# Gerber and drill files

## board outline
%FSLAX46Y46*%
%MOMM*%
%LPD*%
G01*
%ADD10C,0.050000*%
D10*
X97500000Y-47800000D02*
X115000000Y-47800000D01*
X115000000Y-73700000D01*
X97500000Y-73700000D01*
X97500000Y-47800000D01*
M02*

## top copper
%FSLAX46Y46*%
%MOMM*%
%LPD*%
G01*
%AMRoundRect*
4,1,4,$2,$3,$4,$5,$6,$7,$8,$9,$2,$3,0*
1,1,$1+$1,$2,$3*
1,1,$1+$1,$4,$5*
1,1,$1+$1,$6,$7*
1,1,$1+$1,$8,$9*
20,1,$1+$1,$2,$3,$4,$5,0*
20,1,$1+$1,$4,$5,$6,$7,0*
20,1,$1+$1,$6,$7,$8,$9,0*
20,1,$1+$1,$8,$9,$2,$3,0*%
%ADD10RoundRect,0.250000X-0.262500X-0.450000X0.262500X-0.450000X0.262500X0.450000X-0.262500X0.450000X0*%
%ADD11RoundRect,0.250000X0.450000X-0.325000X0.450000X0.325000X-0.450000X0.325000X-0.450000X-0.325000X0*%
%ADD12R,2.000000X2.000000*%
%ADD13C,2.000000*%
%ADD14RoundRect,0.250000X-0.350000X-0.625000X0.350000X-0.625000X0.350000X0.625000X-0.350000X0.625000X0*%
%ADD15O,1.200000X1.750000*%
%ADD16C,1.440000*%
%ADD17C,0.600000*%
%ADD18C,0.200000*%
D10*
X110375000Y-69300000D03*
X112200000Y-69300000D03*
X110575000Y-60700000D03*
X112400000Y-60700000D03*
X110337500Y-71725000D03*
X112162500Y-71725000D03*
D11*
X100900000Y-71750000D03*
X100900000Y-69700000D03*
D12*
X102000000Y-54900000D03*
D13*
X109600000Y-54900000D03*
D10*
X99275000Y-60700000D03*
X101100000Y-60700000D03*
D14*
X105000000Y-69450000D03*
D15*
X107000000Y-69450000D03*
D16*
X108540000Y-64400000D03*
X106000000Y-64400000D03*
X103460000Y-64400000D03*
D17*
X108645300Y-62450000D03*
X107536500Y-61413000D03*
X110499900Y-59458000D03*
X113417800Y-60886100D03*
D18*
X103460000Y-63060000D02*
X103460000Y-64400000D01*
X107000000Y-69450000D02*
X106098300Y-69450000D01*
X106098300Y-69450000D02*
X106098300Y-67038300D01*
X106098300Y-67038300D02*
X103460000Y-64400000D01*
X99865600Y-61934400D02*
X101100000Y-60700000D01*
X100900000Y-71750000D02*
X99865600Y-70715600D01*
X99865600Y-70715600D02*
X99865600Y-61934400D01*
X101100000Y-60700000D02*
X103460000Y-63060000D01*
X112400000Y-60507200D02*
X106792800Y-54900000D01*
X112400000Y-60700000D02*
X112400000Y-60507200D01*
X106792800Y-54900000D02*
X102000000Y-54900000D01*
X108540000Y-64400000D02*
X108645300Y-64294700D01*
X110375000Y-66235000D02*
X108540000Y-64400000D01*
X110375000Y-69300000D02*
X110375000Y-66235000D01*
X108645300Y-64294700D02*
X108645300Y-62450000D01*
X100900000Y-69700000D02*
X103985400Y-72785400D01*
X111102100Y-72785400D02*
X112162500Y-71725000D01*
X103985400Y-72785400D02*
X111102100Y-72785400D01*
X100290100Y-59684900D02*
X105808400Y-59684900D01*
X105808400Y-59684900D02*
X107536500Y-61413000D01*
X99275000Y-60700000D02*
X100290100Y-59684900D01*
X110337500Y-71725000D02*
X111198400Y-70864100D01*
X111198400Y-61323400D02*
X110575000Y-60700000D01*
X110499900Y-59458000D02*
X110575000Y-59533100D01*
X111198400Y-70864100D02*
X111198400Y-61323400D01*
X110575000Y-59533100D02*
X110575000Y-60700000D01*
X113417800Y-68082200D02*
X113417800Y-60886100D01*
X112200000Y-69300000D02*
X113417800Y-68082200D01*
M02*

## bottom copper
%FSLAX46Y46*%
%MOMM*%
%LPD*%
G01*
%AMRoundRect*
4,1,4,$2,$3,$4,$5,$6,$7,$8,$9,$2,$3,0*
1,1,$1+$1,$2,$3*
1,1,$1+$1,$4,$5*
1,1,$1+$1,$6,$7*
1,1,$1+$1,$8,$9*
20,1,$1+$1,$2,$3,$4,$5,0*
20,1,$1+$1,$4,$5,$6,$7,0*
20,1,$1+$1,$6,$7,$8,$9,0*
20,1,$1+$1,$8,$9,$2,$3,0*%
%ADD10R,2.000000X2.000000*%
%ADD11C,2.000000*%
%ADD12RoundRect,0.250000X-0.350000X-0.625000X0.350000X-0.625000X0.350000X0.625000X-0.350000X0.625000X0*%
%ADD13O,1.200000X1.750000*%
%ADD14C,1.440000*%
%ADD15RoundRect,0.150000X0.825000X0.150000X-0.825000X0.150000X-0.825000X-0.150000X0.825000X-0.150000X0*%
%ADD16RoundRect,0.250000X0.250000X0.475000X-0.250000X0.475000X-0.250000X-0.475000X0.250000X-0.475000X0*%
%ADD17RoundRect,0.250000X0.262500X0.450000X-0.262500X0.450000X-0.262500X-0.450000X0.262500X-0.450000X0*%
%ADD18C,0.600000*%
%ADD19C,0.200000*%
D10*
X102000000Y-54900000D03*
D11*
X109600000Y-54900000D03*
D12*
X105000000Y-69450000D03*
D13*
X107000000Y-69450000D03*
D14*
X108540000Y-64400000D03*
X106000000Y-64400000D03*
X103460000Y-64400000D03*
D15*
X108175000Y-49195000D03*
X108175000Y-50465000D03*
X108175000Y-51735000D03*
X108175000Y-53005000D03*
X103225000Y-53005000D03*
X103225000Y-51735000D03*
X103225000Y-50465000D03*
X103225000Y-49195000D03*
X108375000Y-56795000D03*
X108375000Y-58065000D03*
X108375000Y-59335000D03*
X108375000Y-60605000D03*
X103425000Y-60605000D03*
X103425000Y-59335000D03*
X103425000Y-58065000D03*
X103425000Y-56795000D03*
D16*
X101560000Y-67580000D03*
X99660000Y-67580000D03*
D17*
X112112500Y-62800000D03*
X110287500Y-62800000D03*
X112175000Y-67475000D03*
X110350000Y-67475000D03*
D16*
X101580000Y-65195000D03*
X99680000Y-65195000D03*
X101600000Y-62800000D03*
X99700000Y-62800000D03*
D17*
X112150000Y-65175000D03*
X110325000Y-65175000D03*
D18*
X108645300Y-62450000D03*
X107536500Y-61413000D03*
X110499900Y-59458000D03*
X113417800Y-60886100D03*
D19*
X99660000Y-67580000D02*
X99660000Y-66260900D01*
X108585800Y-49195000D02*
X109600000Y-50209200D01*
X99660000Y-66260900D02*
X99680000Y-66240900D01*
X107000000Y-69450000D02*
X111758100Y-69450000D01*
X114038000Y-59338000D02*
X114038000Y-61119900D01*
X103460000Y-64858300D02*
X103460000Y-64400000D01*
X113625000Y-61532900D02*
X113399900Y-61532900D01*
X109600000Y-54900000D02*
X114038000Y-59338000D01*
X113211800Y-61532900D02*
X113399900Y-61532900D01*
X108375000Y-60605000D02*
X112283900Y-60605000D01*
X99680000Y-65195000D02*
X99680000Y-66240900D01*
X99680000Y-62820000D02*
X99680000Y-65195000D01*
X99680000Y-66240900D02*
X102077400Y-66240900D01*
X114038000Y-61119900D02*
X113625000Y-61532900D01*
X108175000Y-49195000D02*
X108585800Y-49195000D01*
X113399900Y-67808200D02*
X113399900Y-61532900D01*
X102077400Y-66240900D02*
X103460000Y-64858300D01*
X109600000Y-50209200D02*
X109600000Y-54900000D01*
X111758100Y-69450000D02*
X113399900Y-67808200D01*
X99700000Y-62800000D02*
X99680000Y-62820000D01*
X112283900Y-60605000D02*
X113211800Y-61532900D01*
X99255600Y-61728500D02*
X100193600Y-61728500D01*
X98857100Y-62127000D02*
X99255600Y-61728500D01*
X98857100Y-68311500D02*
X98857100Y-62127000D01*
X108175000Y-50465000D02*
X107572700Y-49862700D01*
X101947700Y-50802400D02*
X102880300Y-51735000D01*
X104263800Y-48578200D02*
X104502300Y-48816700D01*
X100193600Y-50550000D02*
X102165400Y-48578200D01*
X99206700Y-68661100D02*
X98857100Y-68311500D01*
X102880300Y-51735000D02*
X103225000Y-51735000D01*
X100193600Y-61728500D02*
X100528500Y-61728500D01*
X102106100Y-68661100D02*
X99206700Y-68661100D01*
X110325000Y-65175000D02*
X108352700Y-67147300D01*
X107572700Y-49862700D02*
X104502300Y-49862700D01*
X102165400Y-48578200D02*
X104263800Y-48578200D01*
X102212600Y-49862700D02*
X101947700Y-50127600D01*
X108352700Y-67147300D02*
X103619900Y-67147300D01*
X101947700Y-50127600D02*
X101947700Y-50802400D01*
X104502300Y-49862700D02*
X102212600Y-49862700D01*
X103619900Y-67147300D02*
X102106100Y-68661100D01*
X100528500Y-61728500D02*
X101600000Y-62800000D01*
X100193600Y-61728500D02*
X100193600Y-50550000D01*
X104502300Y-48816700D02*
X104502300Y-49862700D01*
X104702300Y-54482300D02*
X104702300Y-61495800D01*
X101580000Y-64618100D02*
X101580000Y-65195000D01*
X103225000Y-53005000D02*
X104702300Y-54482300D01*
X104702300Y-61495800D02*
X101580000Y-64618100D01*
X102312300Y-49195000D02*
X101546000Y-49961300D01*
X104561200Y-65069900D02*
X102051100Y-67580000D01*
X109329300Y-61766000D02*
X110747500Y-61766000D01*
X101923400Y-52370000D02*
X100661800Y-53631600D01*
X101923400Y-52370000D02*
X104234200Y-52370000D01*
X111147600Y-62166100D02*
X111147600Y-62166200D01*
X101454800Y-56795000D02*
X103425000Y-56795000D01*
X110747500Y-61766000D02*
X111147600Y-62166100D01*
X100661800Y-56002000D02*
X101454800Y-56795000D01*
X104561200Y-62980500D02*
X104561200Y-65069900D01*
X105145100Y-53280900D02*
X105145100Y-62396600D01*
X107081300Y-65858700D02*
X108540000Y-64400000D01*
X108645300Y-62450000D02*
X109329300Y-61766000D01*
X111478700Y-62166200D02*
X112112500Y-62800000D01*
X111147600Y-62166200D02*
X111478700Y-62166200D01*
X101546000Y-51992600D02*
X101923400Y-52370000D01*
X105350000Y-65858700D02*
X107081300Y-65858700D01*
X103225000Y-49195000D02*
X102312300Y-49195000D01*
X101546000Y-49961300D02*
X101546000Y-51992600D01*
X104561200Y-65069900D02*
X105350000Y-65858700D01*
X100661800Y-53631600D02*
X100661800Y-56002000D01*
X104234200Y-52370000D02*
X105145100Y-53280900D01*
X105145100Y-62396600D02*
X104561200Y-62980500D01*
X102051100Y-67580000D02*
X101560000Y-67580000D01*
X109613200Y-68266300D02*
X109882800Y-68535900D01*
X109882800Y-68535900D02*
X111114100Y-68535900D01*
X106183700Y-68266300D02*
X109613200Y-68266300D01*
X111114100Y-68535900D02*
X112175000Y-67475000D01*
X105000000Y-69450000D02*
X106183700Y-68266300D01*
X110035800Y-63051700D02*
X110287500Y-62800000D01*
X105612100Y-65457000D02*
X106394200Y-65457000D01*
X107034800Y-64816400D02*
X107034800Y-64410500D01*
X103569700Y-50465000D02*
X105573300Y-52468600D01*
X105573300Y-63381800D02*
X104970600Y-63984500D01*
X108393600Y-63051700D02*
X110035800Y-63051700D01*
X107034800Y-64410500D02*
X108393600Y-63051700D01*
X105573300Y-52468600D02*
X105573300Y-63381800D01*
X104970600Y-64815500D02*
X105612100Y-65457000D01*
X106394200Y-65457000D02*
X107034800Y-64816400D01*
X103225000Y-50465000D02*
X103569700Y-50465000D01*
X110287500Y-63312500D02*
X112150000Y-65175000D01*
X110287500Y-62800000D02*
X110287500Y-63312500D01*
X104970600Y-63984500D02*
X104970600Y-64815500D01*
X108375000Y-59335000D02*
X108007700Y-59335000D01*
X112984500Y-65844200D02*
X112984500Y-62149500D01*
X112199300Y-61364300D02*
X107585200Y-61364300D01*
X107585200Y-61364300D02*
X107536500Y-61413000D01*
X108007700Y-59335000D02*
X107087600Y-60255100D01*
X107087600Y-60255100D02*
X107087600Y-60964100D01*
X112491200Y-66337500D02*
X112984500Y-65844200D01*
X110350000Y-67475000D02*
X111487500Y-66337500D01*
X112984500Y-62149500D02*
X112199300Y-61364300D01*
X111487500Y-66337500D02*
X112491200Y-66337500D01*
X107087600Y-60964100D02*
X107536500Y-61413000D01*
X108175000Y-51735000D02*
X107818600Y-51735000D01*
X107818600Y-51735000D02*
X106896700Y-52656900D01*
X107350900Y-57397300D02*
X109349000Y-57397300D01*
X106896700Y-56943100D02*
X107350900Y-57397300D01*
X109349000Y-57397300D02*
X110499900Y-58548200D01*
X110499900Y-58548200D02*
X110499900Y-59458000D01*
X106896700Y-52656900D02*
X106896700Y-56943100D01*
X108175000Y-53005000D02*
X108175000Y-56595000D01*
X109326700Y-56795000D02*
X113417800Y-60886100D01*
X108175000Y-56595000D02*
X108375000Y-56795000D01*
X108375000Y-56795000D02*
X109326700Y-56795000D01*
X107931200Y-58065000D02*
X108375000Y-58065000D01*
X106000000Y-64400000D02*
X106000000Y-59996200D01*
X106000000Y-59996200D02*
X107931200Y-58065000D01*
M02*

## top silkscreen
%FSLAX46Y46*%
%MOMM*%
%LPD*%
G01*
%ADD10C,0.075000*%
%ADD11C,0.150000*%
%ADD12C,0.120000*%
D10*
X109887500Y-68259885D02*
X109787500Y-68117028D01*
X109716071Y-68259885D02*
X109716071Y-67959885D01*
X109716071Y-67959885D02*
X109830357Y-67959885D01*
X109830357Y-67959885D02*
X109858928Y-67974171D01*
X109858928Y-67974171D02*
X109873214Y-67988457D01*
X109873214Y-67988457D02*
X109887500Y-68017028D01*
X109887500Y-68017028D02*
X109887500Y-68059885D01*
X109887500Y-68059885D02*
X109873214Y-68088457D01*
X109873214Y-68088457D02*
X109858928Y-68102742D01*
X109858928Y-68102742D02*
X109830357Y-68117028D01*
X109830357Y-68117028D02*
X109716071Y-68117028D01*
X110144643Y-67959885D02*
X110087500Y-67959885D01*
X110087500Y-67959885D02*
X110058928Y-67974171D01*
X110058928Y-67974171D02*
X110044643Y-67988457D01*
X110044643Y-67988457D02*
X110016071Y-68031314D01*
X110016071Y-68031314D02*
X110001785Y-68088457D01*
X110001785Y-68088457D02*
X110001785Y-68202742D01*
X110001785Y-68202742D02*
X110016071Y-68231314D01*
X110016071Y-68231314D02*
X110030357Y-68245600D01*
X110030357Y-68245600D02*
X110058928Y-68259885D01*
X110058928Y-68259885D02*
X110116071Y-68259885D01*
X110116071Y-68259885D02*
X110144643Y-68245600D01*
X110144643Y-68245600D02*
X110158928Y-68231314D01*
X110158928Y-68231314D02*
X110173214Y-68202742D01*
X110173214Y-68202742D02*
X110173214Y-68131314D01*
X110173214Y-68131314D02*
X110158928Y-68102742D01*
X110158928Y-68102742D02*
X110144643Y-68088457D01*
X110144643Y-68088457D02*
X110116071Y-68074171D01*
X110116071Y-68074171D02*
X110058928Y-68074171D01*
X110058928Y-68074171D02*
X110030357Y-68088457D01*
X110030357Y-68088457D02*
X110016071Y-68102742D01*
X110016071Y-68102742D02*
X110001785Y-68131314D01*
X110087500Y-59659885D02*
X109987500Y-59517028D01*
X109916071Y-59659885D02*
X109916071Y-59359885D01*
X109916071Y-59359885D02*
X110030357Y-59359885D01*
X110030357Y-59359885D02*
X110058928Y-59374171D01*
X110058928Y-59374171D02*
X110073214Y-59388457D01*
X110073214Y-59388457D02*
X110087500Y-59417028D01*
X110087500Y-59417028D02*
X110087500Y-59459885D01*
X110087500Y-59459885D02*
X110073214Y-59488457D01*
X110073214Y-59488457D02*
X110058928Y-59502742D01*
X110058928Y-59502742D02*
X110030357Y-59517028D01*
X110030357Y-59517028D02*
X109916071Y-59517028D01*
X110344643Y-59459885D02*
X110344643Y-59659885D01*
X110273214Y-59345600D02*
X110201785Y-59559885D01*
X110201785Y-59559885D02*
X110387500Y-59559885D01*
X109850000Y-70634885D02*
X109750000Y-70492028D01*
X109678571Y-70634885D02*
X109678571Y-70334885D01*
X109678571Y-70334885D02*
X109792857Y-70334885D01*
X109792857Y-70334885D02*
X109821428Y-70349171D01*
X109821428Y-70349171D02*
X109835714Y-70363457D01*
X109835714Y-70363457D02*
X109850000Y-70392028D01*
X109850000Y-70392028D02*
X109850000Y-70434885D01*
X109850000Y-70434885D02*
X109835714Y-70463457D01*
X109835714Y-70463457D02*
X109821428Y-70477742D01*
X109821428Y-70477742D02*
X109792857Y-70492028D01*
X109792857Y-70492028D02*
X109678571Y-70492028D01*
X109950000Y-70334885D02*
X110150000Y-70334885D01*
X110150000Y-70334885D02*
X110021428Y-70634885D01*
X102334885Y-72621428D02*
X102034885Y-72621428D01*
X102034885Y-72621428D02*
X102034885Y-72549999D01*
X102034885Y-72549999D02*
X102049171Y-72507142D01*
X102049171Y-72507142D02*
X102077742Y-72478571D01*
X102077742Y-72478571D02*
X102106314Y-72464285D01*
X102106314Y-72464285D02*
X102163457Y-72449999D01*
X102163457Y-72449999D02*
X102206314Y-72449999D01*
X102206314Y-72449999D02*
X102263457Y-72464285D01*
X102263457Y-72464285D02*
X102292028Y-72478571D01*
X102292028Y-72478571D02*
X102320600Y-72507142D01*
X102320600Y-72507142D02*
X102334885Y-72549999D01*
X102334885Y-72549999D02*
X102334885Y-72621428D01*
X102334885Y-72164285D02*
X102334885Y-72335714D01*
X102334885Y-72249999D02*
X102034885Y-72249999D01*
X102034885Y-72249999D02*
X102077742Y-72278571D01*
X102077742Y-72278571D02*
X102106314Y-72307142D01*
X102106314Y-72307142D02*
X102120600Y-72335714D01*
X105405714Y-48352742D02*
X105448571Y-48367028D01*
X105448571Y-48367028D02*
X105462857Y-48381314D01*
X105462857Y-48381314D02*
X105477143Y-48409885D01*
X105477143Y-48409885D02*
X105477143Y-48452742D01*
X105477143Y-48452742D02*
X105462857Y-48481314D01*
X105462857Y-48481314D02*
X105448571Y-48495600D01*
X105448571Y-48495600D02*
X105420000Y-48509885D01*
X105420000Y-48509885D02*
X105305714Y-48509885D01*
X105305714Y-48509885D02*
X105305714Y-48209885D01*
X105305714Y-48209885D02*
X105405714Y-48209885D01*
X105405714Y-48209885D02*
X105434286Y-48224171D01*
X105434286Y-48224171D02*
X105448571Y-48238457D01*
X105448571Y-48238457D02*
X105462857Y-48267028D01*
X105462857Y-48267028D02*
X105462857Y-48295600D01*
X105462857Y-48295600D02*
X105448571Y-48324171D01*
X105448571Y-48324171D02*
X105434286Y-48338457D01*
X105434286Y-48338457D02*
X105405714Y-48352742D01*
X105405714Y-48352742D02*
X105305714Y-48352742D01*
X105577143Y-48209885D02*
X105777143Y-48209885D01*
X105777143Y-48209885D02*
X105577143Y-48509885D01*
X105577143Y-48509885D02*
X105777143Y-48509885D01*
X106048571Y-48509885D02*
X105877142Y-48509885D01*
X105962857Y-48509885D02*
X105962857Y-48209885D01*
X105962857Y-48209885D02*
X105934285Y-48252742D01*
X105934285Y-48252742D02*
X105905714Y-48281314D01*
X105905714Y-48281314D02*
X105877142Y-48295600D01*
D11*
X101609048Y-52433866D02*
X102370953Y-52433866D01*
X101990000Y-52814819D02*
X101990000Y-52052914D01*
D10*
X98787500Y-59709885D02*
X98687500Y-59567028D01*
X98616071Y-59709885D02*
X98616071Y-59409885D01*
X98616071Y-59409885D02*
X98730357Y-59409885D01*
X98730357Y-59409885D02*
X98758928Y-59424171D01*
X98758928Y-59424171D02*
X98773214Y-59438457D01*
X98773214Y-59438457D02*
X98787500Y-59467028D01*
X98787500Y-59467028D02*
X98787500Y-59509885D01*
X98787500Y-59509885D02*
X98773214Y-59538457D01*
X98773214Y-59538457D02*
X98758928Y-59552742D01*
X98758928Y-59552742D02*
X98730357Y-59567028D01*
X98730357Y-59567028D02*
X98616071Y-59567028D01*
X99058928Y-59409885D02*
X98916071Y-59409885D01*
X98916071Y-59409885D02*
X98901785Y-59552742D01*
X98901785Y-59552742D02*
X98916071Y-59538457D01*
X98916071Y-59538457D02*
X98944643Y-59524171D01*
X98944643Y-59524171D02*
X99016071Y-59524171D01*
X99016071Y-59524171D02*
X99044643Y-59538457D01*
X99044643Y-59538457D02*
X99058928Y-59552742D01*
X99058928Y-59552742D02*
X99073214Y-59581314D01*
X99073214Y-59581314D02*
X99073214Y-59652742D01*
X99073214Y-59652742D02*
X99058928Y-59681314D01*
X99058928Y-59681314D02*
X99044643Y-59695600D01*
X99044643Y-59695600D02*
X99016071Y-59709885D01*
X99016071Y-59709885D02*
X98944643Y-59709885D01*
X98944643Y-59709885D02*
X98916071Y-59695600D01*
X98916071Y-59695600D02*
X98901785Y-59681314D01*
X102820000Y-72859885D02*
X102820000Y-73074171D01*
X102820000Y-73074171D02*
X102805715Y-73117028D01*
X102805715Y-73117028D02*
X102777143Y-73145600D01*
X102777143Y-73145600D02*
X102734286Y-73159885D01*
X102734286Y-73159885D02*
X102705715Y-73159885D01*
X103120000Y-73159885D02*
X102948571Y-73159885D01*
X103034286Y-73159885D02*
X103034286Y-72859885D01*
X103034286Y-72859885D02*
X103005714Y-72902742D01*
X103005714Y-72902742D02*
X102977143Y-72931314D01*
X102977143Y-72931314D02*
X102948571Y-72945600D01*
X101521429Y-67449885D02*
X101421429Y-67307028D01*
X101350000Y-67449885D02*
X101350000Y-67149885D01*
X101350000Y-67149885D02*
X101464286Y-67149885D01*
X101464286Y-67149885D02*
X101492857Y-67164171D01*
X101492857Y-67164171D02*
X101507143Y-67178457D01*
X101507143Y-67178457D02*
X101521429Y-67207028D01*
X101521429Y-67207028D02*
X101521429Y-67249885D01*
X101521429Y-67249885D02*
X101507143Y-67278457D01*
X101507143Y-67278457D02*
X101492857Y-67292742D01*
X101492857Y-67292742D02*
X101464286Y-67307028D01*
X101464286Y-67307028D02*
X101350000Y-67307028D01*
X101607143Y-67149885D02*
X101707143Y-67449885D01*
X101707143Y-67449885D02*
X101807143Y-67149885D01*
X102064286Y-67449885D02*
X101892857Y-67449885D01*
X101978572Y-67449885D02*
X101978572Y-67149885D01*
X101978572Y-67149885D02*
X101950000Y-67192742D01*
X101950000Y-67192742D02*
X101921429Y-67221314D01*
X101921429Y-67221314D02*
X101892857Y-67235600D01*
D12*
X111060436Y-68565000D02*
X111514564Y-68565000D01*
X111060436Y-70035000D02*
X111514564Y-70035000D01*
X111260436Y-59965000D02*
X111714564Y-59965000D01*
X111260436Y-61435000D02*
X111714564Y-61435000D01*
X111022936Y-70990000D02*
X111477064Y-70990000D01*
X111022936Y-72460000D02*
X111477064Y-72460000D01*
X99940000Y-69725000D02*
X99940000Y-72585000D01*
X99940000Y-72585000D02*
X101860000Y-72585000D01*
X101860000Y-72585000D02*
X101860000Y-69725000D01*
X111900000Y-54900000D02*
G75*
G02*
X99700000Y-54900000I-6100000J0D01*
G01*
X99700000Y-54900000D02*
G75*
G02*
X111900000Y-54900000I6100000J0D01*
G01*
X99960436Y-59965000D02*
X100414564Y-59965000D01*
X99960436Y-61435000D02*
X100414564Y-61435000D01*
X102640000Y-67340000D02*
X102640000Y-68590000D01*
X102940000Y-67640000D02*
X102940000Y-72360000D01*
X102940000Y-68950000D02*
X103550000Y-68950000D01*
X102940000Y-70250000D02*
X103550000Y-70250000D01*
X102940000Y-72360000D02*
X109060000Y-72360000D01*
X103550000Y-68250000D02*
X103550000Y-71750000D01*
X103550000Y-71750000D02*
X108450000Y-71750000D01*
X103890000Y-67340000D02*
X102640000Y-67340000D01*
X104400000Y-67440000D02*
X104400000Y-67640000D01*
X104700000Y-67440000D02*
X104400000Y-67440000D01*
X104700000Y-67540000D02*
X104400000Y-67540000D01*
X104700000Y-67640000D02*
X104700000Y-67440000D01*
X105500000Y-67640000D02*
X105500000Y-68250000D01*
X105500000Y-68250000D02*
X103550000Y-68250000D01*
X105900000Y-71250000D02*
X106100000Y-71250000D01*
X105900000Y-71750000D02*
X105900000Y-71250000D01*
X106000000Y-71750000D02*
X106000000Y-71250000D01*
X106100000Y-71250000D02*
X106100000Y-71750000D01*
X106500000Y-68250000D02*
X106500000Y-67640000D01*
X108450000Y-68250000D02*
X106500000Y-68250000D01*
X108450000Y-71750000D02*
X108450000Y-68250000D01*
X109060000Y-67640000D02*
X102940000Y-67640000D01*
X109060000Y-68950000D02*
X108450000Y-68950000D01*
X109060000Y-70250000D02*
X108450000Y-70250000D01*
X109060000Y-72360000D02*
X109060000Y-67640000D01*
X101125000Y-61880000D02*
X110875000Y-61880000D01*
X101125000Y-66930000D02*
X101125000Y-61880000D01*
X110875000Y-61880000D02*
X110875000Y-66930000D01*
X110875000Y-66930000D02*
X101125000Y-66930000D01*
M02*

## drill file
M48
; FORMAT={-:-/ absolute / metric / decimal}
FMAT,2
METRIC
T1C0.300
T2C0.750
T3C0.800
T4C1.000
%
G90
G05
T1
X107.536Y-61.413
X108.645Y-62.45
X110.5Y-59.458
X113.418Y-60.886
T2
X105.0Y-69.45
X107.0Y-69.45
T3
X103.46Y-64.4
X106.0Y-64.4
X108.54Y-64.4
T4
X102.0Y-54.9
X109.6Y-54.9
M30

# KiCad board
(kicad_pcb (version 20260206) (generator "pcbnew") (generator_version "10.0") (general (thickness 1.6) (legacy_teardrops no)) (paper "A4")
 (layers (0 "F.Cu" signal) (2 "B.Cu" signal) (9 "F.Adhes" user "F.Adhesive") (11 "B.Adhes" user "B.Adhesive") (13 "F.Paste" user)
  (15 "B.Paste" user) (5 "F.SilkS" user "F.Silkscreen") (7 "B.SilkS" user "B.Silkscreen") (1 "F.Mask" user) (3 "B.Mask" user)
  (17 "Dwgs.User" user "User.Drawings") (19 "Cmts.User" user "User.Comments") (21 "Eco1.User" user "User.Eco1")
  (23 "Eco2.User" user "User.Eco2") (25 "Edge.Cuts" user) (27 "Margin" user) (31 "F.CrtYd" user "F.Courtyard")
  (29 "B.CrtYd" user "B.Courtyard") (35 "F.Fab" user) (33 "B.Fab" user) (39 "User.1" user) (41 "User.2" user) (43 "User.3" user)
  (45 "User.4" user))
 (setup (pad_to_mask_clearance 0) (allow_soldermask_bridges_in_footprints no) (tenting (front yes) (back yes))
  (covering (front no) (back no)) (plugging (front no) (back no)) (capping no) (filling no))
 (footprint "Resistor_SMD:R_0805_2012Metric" (layer "F.Cu") (at 111.2875 69.3)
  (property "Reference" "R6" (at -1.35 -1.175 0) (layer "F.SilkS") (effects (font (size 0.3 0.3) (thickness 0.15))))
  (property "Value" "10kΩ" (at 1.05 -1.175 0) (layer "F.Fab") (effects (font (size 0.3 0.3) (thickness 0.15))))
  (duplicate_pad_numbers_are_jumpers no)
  (fp_line (start -0.227064 -0.735) (end 0.227064 -0.735) (stroke (width 0.12) (type solid)) (layer "F.SilkS"))
  (fp_line (start -0.227064 0.735) (end 0.227064 0.735) (stroke (width 0.12) (type solid)) (layer "F.SilkS"))
  (pad "1" smd roundrect (at -0.9125 0) (size 1.025 1.4) (layers "F.Cu" "F.Mask" "F.Paste") (roundrect_rratio 0.243902) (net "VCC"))
  (pad "2" smd roundrect (at 0.9125 0) (size 1.025 1.4) (layers "F.Cu" "F.Mask" "F.Paste") (roundrect_rratio 0.243902) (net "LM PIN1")))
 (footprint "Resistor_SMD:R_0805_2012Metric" (layer "F.Cu") (at 111.4875 60.7)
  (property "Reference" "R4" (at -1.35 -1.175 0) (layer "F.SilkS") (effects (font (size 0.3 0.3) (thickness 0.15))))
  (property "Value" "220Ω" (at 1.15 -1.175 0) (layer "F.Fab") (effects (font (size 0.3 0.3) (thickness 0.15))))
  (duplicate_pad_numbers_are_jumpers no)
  (fp_line (start -0.227064 -0.735) (end 0.227064 -0.735) (stroke (width 0.12) (type solid)) (layer "F.SilkS"))
  (fp_line (start -0.227064 0.735) (end 0.227064 0.735) (stroke (width 0.12) (type solid)) (layer "F.SilkS"))
  (pad "1" smd roundrect (at -0.9125 0) (size 1.025 1.4) (layers "F.Cu" "F.Mask" "F.Paste") (roundrect_rratio 0.243902) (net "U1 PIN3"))
  (pad "2" smd roundrect (at 0.9125 0) (size 1.025 1.4) (layers "F.Cu" "F.Mask" "F.Paste") (roundrect_rratio 0.243902) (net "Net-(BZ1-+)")))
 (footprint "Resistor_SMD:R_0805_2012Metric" (layer "F.Cu") (at 111.25 71.725)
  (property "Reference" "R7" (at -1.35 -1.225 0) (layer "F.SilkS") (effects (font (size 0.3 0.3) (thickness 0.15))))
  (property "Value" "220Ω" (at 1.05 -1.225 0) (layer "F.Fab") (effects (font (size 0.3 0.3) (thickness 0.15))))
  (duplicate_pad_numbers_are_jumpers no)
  (fp_line (start -0.227064 -0.735) (end 0.227064 -0.735) (stroke (width 0.12) (type solid)) (layer "F.SilkS"))
  (fp_line (start -0.227064 0.735) (end 0.227064 0.735) (stroke (width 0.12) (type solid)) (layer "F.SilkS"))
  (pad "1" smd roundrect (at -0.9125 0) (size 1.025 1.4) (layers "F.Cu" "F.Mask" "F.Paste") (roundrect_rratio 0.243902) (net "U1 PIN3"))
  (pad "2" smd roundrect (at 0.9125 0) (size 1.025 1.4) (layers "F.Cu" "F.Mask" "F.Paste") (roundrect_rratio 0.243902) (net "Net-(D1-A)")))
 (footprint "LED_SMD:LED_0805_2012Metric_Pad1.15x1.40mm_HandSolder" (layer "F.Cu") (at 100.9 70.725 90)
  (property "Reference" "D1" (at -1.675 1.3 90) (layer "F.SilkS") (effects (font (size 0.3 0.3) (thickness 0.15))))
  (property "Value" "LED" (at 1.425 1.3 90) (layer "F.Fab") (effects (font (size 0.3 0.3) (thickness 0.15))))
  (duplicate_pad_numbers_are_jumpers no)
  (fp_line (start 1 -0.96) (end -1.86 -0.96) (stroke (width 0.12) (type solid)) (layer "F.SilkS"))
  (fp_line (start -1.86 -0.96) (end -1.86 0.96) (stroke (width 0.12) (type solid)) (layer "F.SilkS"))
  (fp_line (start -1.86 0.96) (end 1 0.96) (stroke (width 0.12) (type solid)) (layer "F.SilkS"))
  (pad "1" smd roundrect (at -1.025 0 90) (size 1.15 1.4) (layers "F.Cu" "F.Mask" "F.Paste") (roundrect_rratio 0.217391) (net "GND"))
  (pad "2" smd roundrect (at 1.025 0 90) (size 1.15 1.4) (layers "F.Cu" "F.Mask" "F.Paste") (roundrect_rratio 0.217391) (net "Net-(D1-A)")))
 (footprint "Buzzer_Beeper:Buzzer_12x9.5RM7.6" (layer "F.Cu") (at 102 54.9)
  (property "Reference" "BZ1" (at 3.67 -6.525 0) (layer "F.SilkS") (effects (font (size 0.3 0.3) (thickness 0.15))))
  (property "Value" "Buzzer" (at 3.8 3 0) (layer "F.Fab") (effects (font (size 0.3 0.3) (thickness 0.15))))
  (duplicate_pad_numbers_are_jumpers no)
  (fp_circle (center 3.8 0) (end 9.9 0) (stroke (width 0.12) (type solid)) (fill no) (layer "F.SilkS"))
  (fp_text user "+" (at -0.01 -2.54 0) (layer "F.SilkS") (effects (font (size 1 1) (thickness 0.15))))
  (pad "1" thru_hole rect (at 0 0) (size 2 2) (drill 1) (layers "*.Cu" "*.Mask") (remove_unused_layers no) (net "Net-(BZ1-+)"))
  (pad "2" thru_hole circle (at 7.6 0) (size 2 2) (drill 1) (layers "*.Cu" "*.Mask") (remove_unused_layers no) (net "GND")))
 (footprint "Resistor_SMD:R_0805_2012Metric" (layer "F.Cu") (at 100.1875 60.7)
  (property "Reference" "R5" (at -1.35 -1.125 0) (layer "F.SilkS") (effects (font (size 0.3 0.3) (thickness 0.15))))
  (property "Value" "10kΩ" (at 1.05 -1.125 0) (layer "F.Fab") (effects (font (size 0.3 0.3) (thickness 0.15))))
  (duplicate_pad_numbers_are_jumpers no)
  (fp_line (start -0.227064 -0.735) (end 0.227064 -0.735) (stroke (width 0.12) (type solid)) (layer "F.SilkS"))
  (fp_line (start -0.227064 0.735) (end 0.227064 0.735) (stroke (width 0.12) (type solid)) (layer "F.SilkS"))
  (pad "1" smd roundrect (at -0.9125 0) (size 1.025 1.4) (layers "F.Cu" "F.Mask" "F.Paste") (roundrect_rratio 0.243902)
   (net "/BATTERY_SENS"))
  (pad "2" smd roundrect (at 0.9125 0) (size 1.025 1.4) (layers "F.Cu" "F.Mask" "F.Paste") (roundrect_rratio 0.243902) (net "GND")))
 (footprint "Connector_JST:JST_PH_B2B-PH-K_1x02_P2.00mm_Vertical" (layer "F.Cu") (at 105 69.45)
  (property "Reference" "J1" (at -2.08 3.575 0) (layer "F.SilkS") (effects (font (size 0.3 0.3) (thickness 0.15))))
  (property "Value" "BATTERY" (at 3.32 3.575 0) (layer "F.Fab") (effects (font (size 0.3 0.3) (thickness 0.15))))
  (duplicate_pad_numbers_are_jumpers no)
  (fp_line (start -2.36 -2.11) (end -2.36 -0.86) (stroke (width 0.12) (type solid)) (layer "F.SilkS"))
  (fp_line (start -2.06 -1.81) (end -2.06 2.91) (stroke (width 0.12) (type solid)) (layer "F.SilkS"))
  (fp_line (start -2.06 -0.5) (end -1.45 -0.5) (stroke (width 0.12) (type solid)) (layer "F.SilkS"))
  (fp_line (start -2.06 0.8) (end -1.45 0.8) (stroke (width 0.12) (type solid)) (layer "F.SilkS"))
  (fp_line (start -2.06 2.91) (end 4.06 2.91) (stroke (width 0.12) (type solid)) (layer "F.SilkS"))
  (fp_line (start -1.45 -1.2) (end -1.45 2.3) (stroke (width 0.12) (type solid)) (layer "F.SilkS"))
  (fp_line (start -1.45 2.3) (end 3.45 2.3) (stroke (width 0.12) (type solid)) (layer "F.SilkS"))
  (fp_line (start -1.11 -2.11) (end -2.36 -2.11) (stroke (width 0.12) (type solid)) (layer "F.SilkS"))
  (fp_line (start -0.6 -2.01) (end -0.6 -1.81) (stroke (width 0.12) (type solid)) (layer "F.SilkS"))
  (fp_line (start -0.3 -2.01) (end -0.6 -2.01) (stroke (width 0.12) (type solid)) (layer "F.SilkS"))
  (fp_line (start -0.3 -1.91) (end -0.6 -1.91) (stroke (width 0.12) (type solid)) (layer "F.SilkS"))
  (fp_line (start -0.3 -1.81) (end -0.3 -2.01) (stroke (width 0.12) (type solid)) (layer "F.SilkS"))
  (fp_line (start 0.5 -1.81) (end 0.5 -1.2) (stroke (width 0.12) (type solid)) (layer "F.SilkS"))
  (fp_line (start 0.5 -1.2) (end -1.45 -1.2) (stroke (width 0.12) (type solid)) (layer "F.SilkS"))
  (fp_line (start 0.9 1.8) (end 1.1 1.8) (stroke (width 0.12) (type solid)) (layer "F.SilkS"))
  (fp_line (start 0.9 2.3) (end 0.9 1.8) (stroke (width 0.12) (type solid)) (layer "F.SilkS"))
  (fp_line (start 1 2.3) (end 1 1.8) (stroke (width 0.12) (type solid)) (layer "F.SilkS"))
  (fp_line (start 1.1 1.8) (end 1.1 2.3) (stroke (width 0.12) (type solid)) (layer "F.SilkS"))
  (fp_line (start 1.5 -1.2) (end 1.5 -1.81) (stroke (width 0.12) (type solid)) (layer "F.SilkS"))
  (fp_line (start 3.45 -1.2) (end 1.5 -1.2) (stroke (width 0.12) (type solid)) (layer "F.SilkS"))
  (fp_line (start 3.45 2.3) (end 3.45 -1.2) (stroke (width 0.12) (type solid)) (layer "F.SilkS"))
  (fp_line (start 4.06 -1.81) (end -2.06 -1.81) (stroke (width 0.12) (type solid)) (layer "F.SilkS"))
  (fp_line (start 4.06 -0.5) (end 3.45 -0.5) (stroke (width 0.12) (type solid)) (layer "F.SilkS"))
  (fp_line (start 4.06 0.8) (end 3.45 0.8) (stroke (width 0.12) (type solid)) (layer "F.SilkS"))
  (fp_line (start 4.06 2.91) (end 4.06 -1.81) (stroke (width 0.12) (type solid)) (layer "F.SilkS"))
  (pad "1" thru_hole roundrect (at 0 0) (size 1.2 1.75) (drill 0.75) (layers "*.Cu" "*.Mask") (remove_unused_layers no)
   (roundrect_rratio 0.208333) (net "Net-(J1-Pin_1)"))
  (pad "2" thru_hole oval (at 2 0) (size 1.2 1.75) (drill 0.75) (layers "*.Cu" "*.Mask") (remove_unused_layers no) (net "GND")))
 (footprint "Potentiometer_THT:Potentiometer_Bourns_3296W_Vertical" (layer "F.Cu") (at 108.54 64.4)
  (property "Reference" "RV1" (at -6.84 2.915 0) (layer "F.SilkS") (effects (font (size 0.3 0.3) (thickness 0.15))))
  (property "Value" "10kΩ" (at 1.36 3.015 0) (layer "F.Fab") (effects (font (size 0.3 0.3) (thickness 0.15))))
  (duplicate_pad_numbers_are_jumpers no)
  (fp_line (start -7.415 -2.52) (end 2.335 -2.52) (stroke (width 0.12) (type solid)) (layer "F.SilkS"))
  (fp_line (start -7.415 2.53) (end -7.415 -2.52) (stroke (width 0.12) (type solid)) (layer "F.SilkS"))
  (fp_line (start 2.335 -2.52) (end 2.335 2.53) (stroke (width 0.12) (type solid)) (layer "F.SilkS"))
  (fp_line (start 2.335 2.53) (end -7.415 2.53) (stroke (width 0.12) (type solid)) (layer "F.SilkS"))
  (pad "1" thru_hole circle (at 0 0) (size 1.44 1.44) (drill 0.8) (layers "*.Cu" "*.Mask") (remove_unused_layers no) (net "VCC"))
  (pad "2" thru_hole circle (at -2.54 0) (size 1.44 1.44) (drill 0.8) (layers "*.Cu" "*.Mask") (remove_unused_layers no) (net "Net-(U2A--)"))
  (pad "3" thru_hole circle (at -5.08 0) (size 1.44 1.44) (drill 0.8) (layers "*.Cu" "*.Mask") (remove_unused_layers no) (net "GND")))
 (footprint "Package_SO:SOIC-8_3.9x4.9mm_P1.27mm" (layer "B.Cu") (at 105.7 51.1 180)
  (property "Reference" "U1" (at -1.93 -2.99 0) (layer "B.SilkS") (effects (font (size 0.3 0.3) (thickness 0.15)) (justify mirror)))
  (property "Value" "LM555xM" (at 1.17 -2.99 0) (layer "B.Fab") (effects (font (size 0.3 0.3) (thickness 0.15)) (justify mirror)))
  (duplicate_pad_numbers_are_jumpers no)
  (pad "1" smd roundrect (at -2.475 1.905 180) (size 1.95 0.6) (layers "B.Cu" "B.Mask" "B.Paste") (roundrect_rratio 0.25) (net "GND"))
  (pad "2" smd roundrect (at -2.475 0.635 180) (size 1.95 0.6) (layers "B.Cu" "B.Mask" "B.Paste") (roundrect_rratio 0.25) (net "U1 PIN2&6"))
  (pad "3" smd roundrect (at -2.475 -0.635 180) (size 1.95 0.6) (layers "B.Cu" "B.Mask" "B.Paste") (roundrect_rratio 0.25) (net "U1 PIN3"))
  (pad "4" smd roundrect (at -2.475 -1.905 180) (size 1.95 0.6) (layers "B.Cu" "B.Mask" "B.Paste") (roundrect_rratio 0.25) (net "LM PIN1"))
  (pad "5" smd roundrect (at 2.475 -1.905 180) (size 1.95 0.6) (layers "B.Cu" "B.Mask" "B.Paste") (roundrect_rratio 0.25) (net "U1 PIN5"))
  (pad "6" smd roundrect (at 2.475 -0.635 180) (size 1.95 0.6) (layers "B.Cu" "B.Mask" "B.Paste") (roundrect_rratio 0.25) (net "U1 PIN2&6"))
  (pad "7" smd roundrect (at 2.475 0.635 180) (size 1.95 0.6) (layers "B.Cu" "B.Mask" "B.Paste") (roundrect_rratio 0.25) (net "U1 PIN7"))
  (pad "8" smd roundrect (at 2.475 1.905 180) (size 1.95 0.6) (layers "B.Cu" "B.Mask" "B.Paste") (roundrect_rratio 0.25) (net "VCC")))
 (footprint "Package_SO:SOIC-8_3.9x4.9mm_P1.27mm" (layer "B.Cu") (at 105.9 58.7 180)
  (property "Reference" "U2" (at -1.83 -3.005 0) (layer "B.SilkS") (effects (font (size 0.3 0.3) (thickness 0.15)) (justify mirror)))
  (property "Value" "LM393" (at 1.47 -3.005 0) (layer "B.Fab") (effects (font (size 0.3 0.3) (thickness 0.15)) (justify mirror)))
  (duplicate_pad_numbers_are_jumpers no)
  (pad "1" smd roundrect (at -2.475 1.905 180) (size 1.95 0.6) (layers "B.Cu" "B.Mask" "B.Paste") (roundrect_rratio 0.25) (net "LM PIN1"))
  (pad "2" smd roundrect (at -2.475 0.635 180) (size 1.95 0.6) (layers "B.Cu" "B.Mask" "B.Paste") (roundrect_rratio 0.25)
   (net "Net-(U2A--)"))
  (pad "3" smd roundrect (at -2.475 -0.635 180) (size 1.95 0.6) (layers "B.Cu" "B.Mask" "B.Paste") (roundrect_rratio 0.25)
   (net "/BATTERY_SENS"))
  (pad "4" smd roundrect (at -2.475 -1.905 180) (size 1.95 0.6) (layers "B.Cu" "B.Mask" "B.Paste") (roundrect_rratio 0.25) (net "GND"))
  (pad "5" smd roundrect (at 2.475 -1.905 180) (size 1.95 0.6) (layers "B.Cu" "B.Mask" "B.Paste") (roundrect_rratio 0.25)
   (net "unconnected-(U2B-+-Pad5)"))
  (pad "6" smd roundrect (at 2.475 -0.635 180) (size 1.95 0.6) (layers "B.Cu" "B.Mask" "B.Paste") (roundrect_rratio 0.25)
   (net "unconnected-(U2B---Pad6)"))
  (pad "7" smd roundrect (at 2.475 0.635 180) (size 1.95 0.6) (layers "B.Cu" "B.Mask" "B.Paste") (roundrect_rratio 0.25)
   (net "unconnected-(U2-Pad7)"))
  (pad "8" smd roundrect (at 2.475 1.905 180) (size 1.95 0.6) (layers "B.Cu" "B.Mask" "B.Paste") (roundrect_rratio 0.25) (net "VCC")))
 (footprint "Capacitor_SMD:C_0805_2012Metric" (layer "B.Cu") (at 100.61 67.58 180)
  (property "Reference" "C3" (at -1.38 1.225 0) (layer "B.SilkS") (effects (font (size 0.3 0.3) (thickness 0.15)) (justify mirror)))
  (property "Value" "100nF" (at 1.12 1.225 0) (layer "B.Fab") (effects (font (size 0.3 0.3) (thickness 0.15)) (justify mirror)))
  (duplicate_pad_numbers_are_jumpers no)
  (pad "1" smd roundrect (at -0.95 0 180) (size 1 1.45) (layers "B.Cu" "B.Mask" "B.Paste") (roundrect_rratio 0.25) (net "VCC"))
  (pad "2" smd roundrect (at 0.95 0 180) (size 1 1.45) (layers "B.Cu" "B.Mask" "B.Paste") (roundrect_rratio 0.25) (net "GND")))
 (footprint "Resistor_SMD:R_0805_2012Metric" (layer "B.Cu") (at 111.2 62.8 180)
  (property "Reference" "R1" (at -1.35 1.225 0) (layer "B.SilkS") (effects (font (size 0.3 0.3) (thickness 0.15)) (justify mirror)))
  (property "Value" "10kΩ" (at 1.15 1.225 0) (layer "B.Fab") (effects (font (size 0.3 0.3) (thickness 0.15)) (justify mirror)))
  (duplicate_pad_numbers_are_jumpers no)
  (pad "1" smd roundrect (at -0.9125 0 180) (size 1.025 1.4) (layers "B.Cu" "B.Mask" "B.Paste") (roundrect_rratio 0.243902) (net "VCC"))
  (pad "2" smd roundrect (at 0.9125 0 180) (size 1.025 1.4) (layers "B.Cu" "B.Mask" "B.Paste") (roundrect_rratio 0.243902) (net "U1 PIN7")))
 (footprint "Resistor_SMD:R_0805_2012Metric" (layer "B.Cu") (at 111.2625 67.475 180)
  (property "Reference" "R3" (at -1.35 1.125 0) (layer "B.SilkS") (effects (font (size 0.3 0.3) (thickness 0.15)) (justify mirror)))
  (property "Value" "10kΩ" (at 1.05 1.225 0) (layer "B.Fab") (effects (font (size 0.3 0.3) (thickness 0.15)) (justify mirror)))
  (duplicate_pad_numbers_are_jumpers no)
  (pad "1" smd roundrect (at -0.9125 0 180) (size 1.025 1.4) (layers "B.Cu" "B.Mask" "B.Paste") (roundrect_rratio 0.243902)
   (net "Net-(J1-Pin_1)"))
  (pad "2" smd roundrect (at 0.9125 0 180) (size 1.025 1.4) (layers "B.Cu" "B.Mask" "B.Paste") (roundrect_rratio 0.243902)
   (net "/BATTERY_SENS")))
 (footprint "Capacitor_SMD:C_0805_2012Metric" (layer "B.Cu") (at 100.63 65.195 180)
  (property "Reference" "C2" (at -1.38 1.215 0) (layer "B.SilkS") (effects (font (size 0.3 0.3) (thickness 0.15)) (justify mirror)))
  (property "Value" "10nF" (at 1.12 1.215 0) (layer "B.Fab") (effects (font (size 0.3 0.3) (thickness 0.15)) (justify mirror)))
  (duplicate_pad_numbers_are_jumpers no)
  (pad "1" smd roundrect (at -0.95 0 180) (size 1 1.45) (layers "B.Cu" "B.Mask" "B.Paste") (roundrect_rratio 0.25) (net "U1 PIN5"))
  (pad "2" smd roundrect (at 0.95 0 180) (size 1 1.45) (layers "B.Cu" "B.Mask" "B.Paste") (roundrect_rratio 0.25) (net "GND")))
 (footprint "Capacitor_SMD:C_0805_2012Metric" (layer "B.Cu") (at 100.65 62.8 180)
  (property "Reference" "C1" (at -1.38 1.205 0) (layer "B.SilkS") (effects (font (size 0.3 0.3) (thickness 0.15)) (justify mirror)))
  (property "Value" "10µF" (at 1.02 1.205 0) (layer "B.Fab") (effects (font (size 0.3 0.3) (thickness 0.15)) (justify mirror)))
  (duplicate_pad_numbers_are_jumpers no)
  (pad "1" smd roundrect (at -0.95 0 180) (size 1 1.45) (layers "B.Cu" "B.Mask" "B.Paste") (roundrect_rratio 0.25) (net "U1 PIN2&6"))
  (pad "2" smd roundrect (at 0.95 0 180) (size 1 1.45) (layers "B.Cu" "B.Mask" "B.Paste") (roundrect_rratio 0.25) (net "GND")))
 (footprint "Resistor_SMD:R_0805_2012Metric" (layer "B.Cu") (at 111.2375 65.175 180)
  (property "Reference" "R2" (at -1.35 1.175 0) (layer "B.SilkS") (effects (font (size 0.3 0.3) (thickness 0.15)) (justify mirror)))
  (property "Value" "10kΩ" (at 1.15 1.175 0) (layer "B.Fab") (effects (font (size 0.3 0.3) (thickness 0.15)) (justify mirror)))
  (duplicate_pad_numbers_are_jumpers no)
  (pad "1" smd roundrect (at -0.9125 0 180) (size 1.025 1.4) (layers "B.Cu" "B.Mask" "B.Paste") (roundrect_rratio 0.243902) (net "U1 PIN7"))
  (pad "2" smd roundrect (at 0.9125 0 180) (size 1.025 1.4) (layers "B.Cu" "B.Mask" "B.Paste") (roundrect_rratio 0.243902) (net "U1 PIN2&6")))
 (gr_rect (start 97.5 47.8) (end 115 73.7) (stroke (width 0.05) (type default)) (fill no) (layer "Edge.Cuts"))
 (segment (start 103.46 63.06) (end 103.46 64.4) (width 0.2) (layer "F.Cu") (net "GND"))
 (segment (start 107 69.45) (end 106.0983 69.45) (width 0.2) (layer "F.Cu") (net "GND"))
 (segment (start 106.0983 69.45) (end 106.0983 67.0383) (width 0.2) (layer "F.Cu") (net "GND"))
 (segment (start 106.0983 67.0383) (end 103.46 64.4) (width 0.2) (layer "F.Cu") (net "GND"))
 (segment (start 99.8656 61.9344) (end 101.1 60.7) (width 0.2) (layer "F.Cu") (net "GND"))
 (segment (start 100.9 71.75) (end 99.8656 70.7156) (width 0.2) (layer "F.Cu") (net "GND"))
 (segment (start 99.8656 70.7156) (end 99.8656 61.9344) (width 0.2) (layer "F.Cu") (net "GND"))
 (segment (start 101.1 60.7) (end 103.46 63.06) (width 0.2) (layer "F.Cu") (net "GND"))
 (segment (start 99.66 67.58) (end 99.66 66.2609) (width 0.2) (layer "B.Cu") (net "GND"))
 (segment (start 108.5858 49.195) (end 109.6 50.2092) (width 0.2) (layer "B.Cu") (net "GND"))
 (segment (start 99.66 66.2609) (end 99.68 66.2409) (width 0.2) (layer "B.Cu") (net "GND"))
 (segment (start 107 69.45) (end 111.7581 69.45) (width 0.2) (layer "B.Cu") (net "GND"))
 (segment (start 114.038 59.338) (end 114.038 61.1199) (width 0.2) (layer "B.Cu") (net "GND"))
 (segment (start 103.46 64.8583) (end 103.46 64.4) (width 0.2) (layer "B.Cu") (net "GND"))
 (segment (start 113.625 61.5329) (end 113.3999 61.5329) (width 0.2) (layer "B.Cu") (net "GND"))
 (segment (start 109.6 54.9) (end 114.038 59.338) (width 0.2) (layer "B.Cu") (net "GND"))
 (segment (start 113.2118 61.5329) (end 113.3999 61.5329) (width 0.2) (layer "B.Cu") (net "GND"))
 (segment (start 108.375 60.605) (end 112.2839 60.605) (width 0.2) (layer "B.Cu") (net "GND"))
 (segment (start 99.68 65.195) (end 99.68 66.2409) (width 0.2) (layer "B.Cu") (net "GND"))
 (segment (start 99.68 62.82) (end 99.68 65.195) (width 0.2) (layer "B.Cu") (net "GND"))
 (segment (start 99.68 66.2409) (end 102.0774 66.2409) (width 0.2) (layer "B.Cu") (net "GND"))
 (segment (start 114.038 61.1199) (end 113.625 61.5329) (width 0.2) (layer "B.Cu") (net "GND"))
 (segment (start 108.175 49.195) (end 108.5858 49.195) (width 0.2) (layer "B.Cu") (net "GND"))
 (segment (start 113.3999 67.8082) (end 113.3999 61.5329) (width 0.2) (layer "B.Cu") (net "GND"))
 (segment (start 102.0774 66.2409) (end 103.46 64.8583) (width 0.2) (layer "B.Cu") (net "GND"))
 (segment (start 109.6 50.2092) (end 109.6 54.9) (width 0.2) (layer "B.Cu") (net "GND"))
 (segment (start 111.7581 69.45) (end 113.3999 67.8082) (width 0.2) (layer "B.Cu") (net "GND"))
 (segment (start 99.7 62.8) (end 99.68 62.82) (width 0.2) (layer "B.Cu") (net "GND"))
 (segment (start 112.2839 60.605) (end 113.2118 61.5329) (width 0.2) (layer "B.Cu") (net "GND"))
 (segment (start 112.4 60.5072) (end 106.7928 54.9) (width 0.2) (layer "F.Cu") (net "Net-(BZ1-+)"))
 (segment (start 112.4 60.7) (end 112.4 60.5072) (width 0.2) (layer "F.Cu") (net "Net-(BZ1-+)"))
 (segment (start 106.7928 54.9) (end 102 54.9) (width 0.2) (layer "F.Cu") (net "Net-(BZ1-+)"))
 (segment (start 99.2556 61.7285) (end 100.1936 61.7285) (width 0.2) (layer "B.Cu") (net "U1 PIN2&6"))
 (segment (start 98.8571 62.127) (end 99.2556 61.7285) (width 0.2) (layer "B.Cu") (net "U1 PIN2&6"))
 (segment (start 98.8571 68.3115) (end 98.8571 62.127) (width 0.2) (layer "B.Cu") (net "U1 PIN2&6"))
 (segment (start 108.175 50.465) (end 107.5727 49.8627) (width 0.2) (layer "B.Cu") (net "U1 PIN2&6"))
 (segment (start 101.9477 50.8024) (end 102.8803 51.735) (width 0.2) (layer "B.Cu") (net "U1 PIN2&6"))
 (segment (start 104.2638 48.5782) (end 104.5023 48.8167) (width 0.2) (layer "B.Cu") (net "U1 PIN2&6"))
 (segment (start 100.1936 50.55) (end 102.1654 48.5782) (width 0.2) (layer "B.Cu") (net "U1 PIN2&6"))
 (segment (start 99.2067 68.6611) (end 98.8571 68.3115) (width 0.2) (layer "B.Cu") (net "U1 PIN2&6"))
 (segment (start 102.8803 51.735) (end 103.225 51.735) (width 0.2) (layer "B.Cu") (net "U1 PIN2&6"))
 (segment (start 100.1936 61.7285) (end 100.5285 61.7285) (width 0.2) (layer "B.Cu") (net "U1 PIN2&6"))
 (segment (start 102.1061 68.6611) (end 99.2067 68.6611) (width 0.2) (layer "B.Cu") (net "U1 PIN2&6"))
 (segment (start 110.325 65.175) (end 108.3527 67.1473) (width 0.2) (layer "B.Cu") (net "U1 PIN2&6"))
 (segment (start 107.5727 49.8627) (end 104.5023 49.8627) (width 0.2) (layer "B.Cu") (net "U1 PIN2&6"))
 (segment (start 102.1654 48.5782) (end 104.2638 48.5782) (width 0.2) (layer "B.Cu") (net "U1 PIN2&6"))
 (segment (start 102.2126 49.8627) (end 101.9477 50.1276) (width 0.2) (layer "B.Cu") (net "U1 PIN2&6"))
 (segment (start 108.3527 67.1473) (end 103.6199 67.1473) (width 0.2) (layer "B.Cu") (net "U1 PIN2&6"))
 (segment (start 101.9477 50.1276) (end 101.9477 50.8024) (width 0.2) (layer "B.Cu") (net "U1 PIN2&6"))
 (segment (start 104.5023 49.8627) (end 102.2126 49.8627) (width 0.2) (layer "B.Cu") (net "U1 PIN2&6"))
 (segment (start 103.6199 67.1473) (end 102.1061 68.6611) (width 0.2) (layer "B.Cu") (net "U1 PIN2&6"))
 (segment (start 100.5285 61.7285) (end 101.6 62.8) (width 0.2) (layer "B.Cu") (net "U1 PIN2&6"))
 (segment (start 100.1936 61.7285) (end 100.1936 50.55) (width 0.2) (layer "B.Cu") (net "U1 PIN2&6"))
 (segment (start 104.5023 48.8167) (end 104.5023 49.8627) (width 0.2) (layer "B.Cu") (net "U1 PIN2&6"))
 (segment (start 104.7023 54.4823) (end 104.7023 61.4958) (width 0.2) (layer "B.Cu") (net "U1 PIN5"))
 (segment (start 101.58 64.6181) (end 101.58 65.195) (width 0.2) (layer "B.Cu") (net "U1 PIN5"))
 (segment (start 103.225 53.005) (end 104.7023 54.4823) (width 0.2) (layer "B.Cu") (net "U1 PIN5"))
 (segment (start 104.7023 61.4958) (end 101.58 64.6181) (width 0.2) (layer "B.Cu") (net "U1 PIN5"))
 (segment (start 108.54 64.4) (end 108.6453 64.2947) (width 0.2) (layer "F.Cu") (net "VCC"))
 (segment (start 110.375 66.235) (end 108.54 64.4) (width 0.2) (layer "F.Cu") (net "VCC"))
 (segment (start 110.375 69.3) (end 110.375 66.235) (width 0.2) (layer "F.Cu") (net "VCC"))
 (segment (start 108.6453 64.2947) (end 108.6453 62.45) (width 0.2) (layer "F.Cu") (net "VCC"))
 (via (at 108.6453 62.45) (size 0.6) (drill 0.3) (layers "F.Cu" "B.Cu") (capping no) (covering (front no) (back no))
  (plugging (front no) (back no)) (filling no) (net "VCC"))
 (segment (start 102.3123 49.195) (end 101.546 49.9613) (width 0.2) (layer "B.Cu") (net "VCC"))
 (segment (start 104.5612 65.0699) (end 102.0511 67.58) (width 0.2) (layer "B.Cu") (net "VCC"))
 (segment (start 109.3293 61.766) (end 110.7475 61.766) (width 0.2) (layer "B.Cu") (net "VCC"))
 (segment (start 101.9234 52.37) (end 100.6618 53.6316) (width 0.2) (layer "B.Cu") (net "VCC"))
 (segment (start 101.9234 52.37) (end 104.2342 52.37) (width 0.2) (layer "B.Cu") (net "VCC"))
 (segment (start 111.1476 62.1661) (end 111.1476 62.1662) (width 0.2) (layer "B.Cu") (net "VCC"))
 (segment (start 101.4548 56.795) (end 103.425 56.795) (width 0.2) (layer "B.Cu") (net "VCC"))
 (segment (start 110.7475 61.766) (end 111.1476 62.1661) (width 0.2) (layer "B.Cu") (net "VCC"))
 (segment (start 100.6618 56.002) (end 101.4548 56.795) (width 0.2) (layer "B.Cu") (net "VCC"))
 (segment (start 104.5612 62.9805) (end 104.5612 65.0699) (width 0.2) (layer "B.Cu") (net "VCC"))
 (segment (start 105.1451 53.2809) (end 105.1451 62.3966) (width 0.2) (layer "B.Cu") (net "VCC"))
 (segment (start 107.0813 65.8587) (end 108.54 64.4) (width 0.2) (layer "B.Cu") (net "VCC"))
 (segment (start 108.6453 62.45) (end 109.3293 61.766) (width 0.2) (layer "B.Cu") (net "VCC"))
 (segment (start 111.4787 62.1662) (end 112.1125 62.8) (width 0.2) (layer "B.Cu") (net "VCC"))
 (segment (start 111.1476 62.1662) (end 111.4787 62.1662) (width 0.2) (layer "B.Cu") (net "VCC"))
 (segment (start 101.546 51.9926) (end 101.9234 52.37) (width 0.2) (layer "B.Cu") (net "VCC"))
 (segment (start 105.35 65.8587) (end 107.0813 65.8587) (width 0.2) (layer "B.Cu") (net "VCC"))
 (segment (start 103.225 49.195) (end 102.3123 49.195) (width 0.2) (layer "B.Cu") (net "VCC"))
 (segment (start 101.546 49.9613) (end 101.546 51.9926) (width 0.2) (layer "B.Cu") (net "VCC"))
 (segment (start 104.5612 65.0699) (end 105.35 65.8587) (width 0.2) (layer "B.Cu") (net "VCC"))
 (segment (start 100.6618 53.6316) (end 100.6618 56.002) (width 0.2) (layer "B.Cu") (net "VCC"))
 (segment (start 104.2342 52.37) (end 105.1451 53.2809) (width 0.2) (layer "B.Cu") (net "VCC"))
 (segment (start 105.1451 62.3966) (end 104.5612 62.9805) (width 0.2) (layer "B.Cu") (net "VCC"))
 (segment (start 102.0511 67.58) (end 101.56 67.58) (width 0.2) (layer "B.Cu") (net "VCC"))
 (segment (start 100.9 69.7) (end 103.9854 72.7854) (width 0.2) (layer "F.Cu") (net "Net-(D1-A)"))
 (segment (start 111.1021 72.7854) (end 112.1625 71.725) (width 0.2) (layer "F.Cu") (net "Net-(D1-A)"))
 (segment (start 103.9854 72.7854) (end 111.1021 72.7854) (width 0.2) (layer "F.Cu") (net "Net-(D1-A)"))
 (segment (start 109.6132 68.2663) (end 109.8828 68.5359) (width 0.2) (layer "B.Cu") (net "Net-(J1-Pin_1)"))
 (segment (start 109.8828 68.5359) (end 111.1141 68.5359) (width 0.2) (layer "B.Cu") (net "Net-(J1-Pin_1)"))
 (segment (start 106.1837 68.2663) (end 109.6132 68.2663) (width 0.2) (layer "B.Cu") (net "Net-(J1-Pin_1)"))
 (segment (start 111.1141 68.5359) (end 112.175 67.475) (width 0.2) (layer "B.Cu") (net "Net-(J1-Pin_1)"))
 (segment (start 105 69.45) (end 106.1837 68.2663) (width 0.2) (layer "B.Cu") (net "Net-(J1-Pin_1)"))
 (segment (start 110.0358 63.0517) (end 110.2875 62.8) (width 0.2) (layer "B.Cu") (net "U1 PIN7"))
 (segment (start 105.6121 65.457) (end 106.3942 65.457) (width 0.2) (layer "B.Cu") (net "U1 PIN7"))
 (segment (start 107.0348 64.8164) (end 107.0348 64.4105) (width 0.2) (layer "B.Cu") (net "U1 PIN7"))
 (segment (start 103.5697 50.465) (end 105.5733 52.4686) (width 0.2) (layer "B.Cu") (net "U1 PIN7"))
 (segment (start 105.5733 63.3818) (end 104.9706 63.9845) (width 0.2) (layer "B.Cu") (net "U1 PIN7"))
 (segment (start 108.3936 63.0517) (end 110.0358 63.0517) (width 0.2) (layer "B.Cu") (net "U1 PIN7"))
 (segment (start 107.0348 64.4105) (end 108.3936 63.0517) (width 0.2) (layer "B.Cu") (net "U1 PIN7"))
 (segment (start 105.5733 52.4686) (end 105.5733 63.3818) (width 0.2) (layer "B.Cu") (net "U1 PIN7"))
 (segment (start 104.9706 64.8155) (end 105.6121 65.457) (width 0.2) (layer "B.Cu") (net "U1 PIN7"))
 (segment (start 106.3942 65.457) (end 107.0348 64.8164) (width 0.2) (layer "B.Cu") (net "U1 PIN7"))
 (segment (start 103.225 50.465) (end 103.5697 50.465) (width 0.2) (layer "B.Cu") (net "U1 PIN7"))
 (segment (start 110.2875 63.3125) (end 112.15 65.175) (width 0.2) (layer "B.Cu") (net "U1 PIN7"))
 (segment (start 110.2875 62.8) (end 110.2875 63.3125) (width 0.2) (layer "B.Cu") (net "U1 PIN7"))
 (segment (start 104.9706 63.9845) (end 104.9706 64.8155) (width 0.2) (layer "B.Cu") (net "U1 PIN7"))
 (segment (start 100.2901 59.6849) (end 105.8084 59.6849) (width 0.2) (layer "F.Cu") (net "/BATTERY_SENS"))
 (segment (start 105.8084 59.6849) (end 107.5365 61.413) (width 0.2) (layer "F.Cu") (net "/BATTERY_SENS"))
 (segment (start 99.275 60.7) (end 100.2901 59.6849) (width 0.2) (layer "F.Cu") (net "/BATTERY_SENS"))
 (via (at 107.5365 61.413) (size 0.6) (drill 0.3) (layers "F.Cu" "B.Cu") (capping no) (covering (front no) (back no))
  (plugging (front no) (back no)) (filling no) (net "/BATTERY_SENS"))
 (segment (start 108.375 59.335) (end 108.0077 59.335) (width 0.2) (layer "B.Cu") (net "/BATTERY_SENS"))
 (segment (start 112.9845 65.8442) (end 112.9845 62.1495) (width 0.2) (layer "B.Cu") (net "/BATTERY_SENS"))
 (segment (start 112.1993 61.3643) (end 107.5852 61.3643) (width 0.2) (layer "B.Cu") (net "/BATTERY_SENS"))
 (segment (start 107.5852 61.3643) (end 107.5365 61.413) (width 0.2) (layer "B.Cu") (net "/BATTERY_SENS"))
 (segment (start 108.0077 59.335) (end 107.0876 60.2551) (width 0.2) (layer "B.Cu") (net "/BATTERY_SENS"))
 (segment (start 107.0876 60.2551) (end 107.0876 60.9641) (width 0.2) (layer "B.Cu") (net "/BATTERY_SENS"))
 (segment (start 112.4912 66.3375) (end 112.9845 65.8442) (width 0.2) (layer "B.Cu") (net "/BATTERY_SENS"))
 (segment (start 110.35 67.475) (end 111.4875 66.3375) (width 0.2) (layer "B.Cu") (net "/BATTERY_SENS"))
 (segment (start 112.9845 62.1495) (end 112.1993 61.3643) (width 0.2) (layer "B.Cu") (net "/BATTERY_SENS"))
 (segment (start 111.4875 66.3375) (end 112.4912 66.3375) (width 0.2) (layer "B.Cu") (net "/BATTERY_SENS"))
 (segment (start 107.0876 60.9641) (end 107.5365 61.413) (width 0.2) (layer "B.Cu") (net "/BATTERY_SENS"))
 (segment (start 110.3375 71.725) (end 111.1984 70.8641) (width 0.2) (layer "F.Cu") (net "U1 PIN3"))
 (segment (start 111.1984 61.3234) (end 110.575 60.7) (width 0.2) (layer "F.Cu") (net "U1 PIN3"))
 (segment (start 110.4999 59.458) (end 110.575 59.5331) (width 0.2) (layer "F.Cu") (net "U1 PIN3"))
 (segment (start 111.1984 70.8641) (end 111.1984 61.3234) (width 0.2) (layer "F.Cu") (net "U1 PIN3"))
 (segment (start 110.575 59.5331) (end 110.575 60.7) (width 0.2) (layer "F.Cu") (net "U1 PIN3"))
 (via (at 110.4999 59.458) (size 0.6) (drill 0.3) (layers "F.Cu" "B.Cu") (capping no) (covering (front no) (back no))
  (plugging (front no) (back no)) (filling no) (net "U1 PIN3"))
 (segment (start 108.175 51.735) (end 107.8186 51.735) (width 0.2) (layer "B.Cu") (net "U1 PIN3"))
 (segment (start 107.8186 51.735) (end 106.8967 52.6569) (width 0.2) (layer "B.Cu") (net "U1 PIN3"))
 (segment (start 107.3509 57.3973) (end 109.349 57.3973) (width 0.2) (layer "B.Cu") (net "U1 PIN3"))
 (segment (start 106.8967 56.9431) (end 107.3509 57.3973) (width 0.2) (layer "B.Cu") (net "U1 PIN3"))
 (segment (start 109.349 57.3973) (end 110.4999 58.5482) (width 0.2) (layer "B.Cu") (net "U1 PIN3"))
 (segment (start 110.4999 58.5482) (end 110.4999 59.458) (width 0.2) (layer "B.Cu") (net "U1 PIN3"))
 (segment (start 106.8967 52.6569) (end 106.8967 56.9431) (width 0.2) (layer "B.Cu") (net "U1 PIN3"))
 (segment (start 113.4178 68.0822) (end 113.4178 60.8861) (width 0.2) (layer "F.Cu") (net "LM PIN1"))
 (segment (start 112.2 69.3) (end 113.4178 68.0822) (width 0.2) (layer "F.Cu") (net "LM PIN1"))
 (via (at 113.4178 60.8861) (size 0.6) (drill 0.3) (layers "F.Cu" "B.Cu") (capping no) (covering (front no) (back no))
  (plugging (front no) (back no)) (filling no) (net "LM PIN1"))
 (segment (start 108.175 53.005) (end 108.175 56.595) (width 0.2) (layer "B.Cu") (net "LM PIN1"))
 (segment (start 109.3267 56.795) (end 113.4178 60.8861) (width 0.2) (layer "B.Cu") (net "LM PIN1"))
 (segment (start 108.175 56.595) (end 108.375 56.795) (width 0.2) (layer "B.Cu") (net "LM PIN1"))
 (segment (start 108.375 56.795) (end 109.3267 56.795) (width 0.2) (layer "B.Cu") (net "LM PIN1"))
 (segment (start 107.9312 58.065) (end 108.375 58.065) (width 0.2) (layer "B.Cu") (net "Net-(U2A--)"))
 (segment (start 106 64.4) (end 106 59.9962) (width 0.2) (layer "B.Cu") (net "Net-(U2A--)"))
 (segment (start 106 59.9962) (end 107.9312 58.065) (width 0.2) (layer "B.Cu") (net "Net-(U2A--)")))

